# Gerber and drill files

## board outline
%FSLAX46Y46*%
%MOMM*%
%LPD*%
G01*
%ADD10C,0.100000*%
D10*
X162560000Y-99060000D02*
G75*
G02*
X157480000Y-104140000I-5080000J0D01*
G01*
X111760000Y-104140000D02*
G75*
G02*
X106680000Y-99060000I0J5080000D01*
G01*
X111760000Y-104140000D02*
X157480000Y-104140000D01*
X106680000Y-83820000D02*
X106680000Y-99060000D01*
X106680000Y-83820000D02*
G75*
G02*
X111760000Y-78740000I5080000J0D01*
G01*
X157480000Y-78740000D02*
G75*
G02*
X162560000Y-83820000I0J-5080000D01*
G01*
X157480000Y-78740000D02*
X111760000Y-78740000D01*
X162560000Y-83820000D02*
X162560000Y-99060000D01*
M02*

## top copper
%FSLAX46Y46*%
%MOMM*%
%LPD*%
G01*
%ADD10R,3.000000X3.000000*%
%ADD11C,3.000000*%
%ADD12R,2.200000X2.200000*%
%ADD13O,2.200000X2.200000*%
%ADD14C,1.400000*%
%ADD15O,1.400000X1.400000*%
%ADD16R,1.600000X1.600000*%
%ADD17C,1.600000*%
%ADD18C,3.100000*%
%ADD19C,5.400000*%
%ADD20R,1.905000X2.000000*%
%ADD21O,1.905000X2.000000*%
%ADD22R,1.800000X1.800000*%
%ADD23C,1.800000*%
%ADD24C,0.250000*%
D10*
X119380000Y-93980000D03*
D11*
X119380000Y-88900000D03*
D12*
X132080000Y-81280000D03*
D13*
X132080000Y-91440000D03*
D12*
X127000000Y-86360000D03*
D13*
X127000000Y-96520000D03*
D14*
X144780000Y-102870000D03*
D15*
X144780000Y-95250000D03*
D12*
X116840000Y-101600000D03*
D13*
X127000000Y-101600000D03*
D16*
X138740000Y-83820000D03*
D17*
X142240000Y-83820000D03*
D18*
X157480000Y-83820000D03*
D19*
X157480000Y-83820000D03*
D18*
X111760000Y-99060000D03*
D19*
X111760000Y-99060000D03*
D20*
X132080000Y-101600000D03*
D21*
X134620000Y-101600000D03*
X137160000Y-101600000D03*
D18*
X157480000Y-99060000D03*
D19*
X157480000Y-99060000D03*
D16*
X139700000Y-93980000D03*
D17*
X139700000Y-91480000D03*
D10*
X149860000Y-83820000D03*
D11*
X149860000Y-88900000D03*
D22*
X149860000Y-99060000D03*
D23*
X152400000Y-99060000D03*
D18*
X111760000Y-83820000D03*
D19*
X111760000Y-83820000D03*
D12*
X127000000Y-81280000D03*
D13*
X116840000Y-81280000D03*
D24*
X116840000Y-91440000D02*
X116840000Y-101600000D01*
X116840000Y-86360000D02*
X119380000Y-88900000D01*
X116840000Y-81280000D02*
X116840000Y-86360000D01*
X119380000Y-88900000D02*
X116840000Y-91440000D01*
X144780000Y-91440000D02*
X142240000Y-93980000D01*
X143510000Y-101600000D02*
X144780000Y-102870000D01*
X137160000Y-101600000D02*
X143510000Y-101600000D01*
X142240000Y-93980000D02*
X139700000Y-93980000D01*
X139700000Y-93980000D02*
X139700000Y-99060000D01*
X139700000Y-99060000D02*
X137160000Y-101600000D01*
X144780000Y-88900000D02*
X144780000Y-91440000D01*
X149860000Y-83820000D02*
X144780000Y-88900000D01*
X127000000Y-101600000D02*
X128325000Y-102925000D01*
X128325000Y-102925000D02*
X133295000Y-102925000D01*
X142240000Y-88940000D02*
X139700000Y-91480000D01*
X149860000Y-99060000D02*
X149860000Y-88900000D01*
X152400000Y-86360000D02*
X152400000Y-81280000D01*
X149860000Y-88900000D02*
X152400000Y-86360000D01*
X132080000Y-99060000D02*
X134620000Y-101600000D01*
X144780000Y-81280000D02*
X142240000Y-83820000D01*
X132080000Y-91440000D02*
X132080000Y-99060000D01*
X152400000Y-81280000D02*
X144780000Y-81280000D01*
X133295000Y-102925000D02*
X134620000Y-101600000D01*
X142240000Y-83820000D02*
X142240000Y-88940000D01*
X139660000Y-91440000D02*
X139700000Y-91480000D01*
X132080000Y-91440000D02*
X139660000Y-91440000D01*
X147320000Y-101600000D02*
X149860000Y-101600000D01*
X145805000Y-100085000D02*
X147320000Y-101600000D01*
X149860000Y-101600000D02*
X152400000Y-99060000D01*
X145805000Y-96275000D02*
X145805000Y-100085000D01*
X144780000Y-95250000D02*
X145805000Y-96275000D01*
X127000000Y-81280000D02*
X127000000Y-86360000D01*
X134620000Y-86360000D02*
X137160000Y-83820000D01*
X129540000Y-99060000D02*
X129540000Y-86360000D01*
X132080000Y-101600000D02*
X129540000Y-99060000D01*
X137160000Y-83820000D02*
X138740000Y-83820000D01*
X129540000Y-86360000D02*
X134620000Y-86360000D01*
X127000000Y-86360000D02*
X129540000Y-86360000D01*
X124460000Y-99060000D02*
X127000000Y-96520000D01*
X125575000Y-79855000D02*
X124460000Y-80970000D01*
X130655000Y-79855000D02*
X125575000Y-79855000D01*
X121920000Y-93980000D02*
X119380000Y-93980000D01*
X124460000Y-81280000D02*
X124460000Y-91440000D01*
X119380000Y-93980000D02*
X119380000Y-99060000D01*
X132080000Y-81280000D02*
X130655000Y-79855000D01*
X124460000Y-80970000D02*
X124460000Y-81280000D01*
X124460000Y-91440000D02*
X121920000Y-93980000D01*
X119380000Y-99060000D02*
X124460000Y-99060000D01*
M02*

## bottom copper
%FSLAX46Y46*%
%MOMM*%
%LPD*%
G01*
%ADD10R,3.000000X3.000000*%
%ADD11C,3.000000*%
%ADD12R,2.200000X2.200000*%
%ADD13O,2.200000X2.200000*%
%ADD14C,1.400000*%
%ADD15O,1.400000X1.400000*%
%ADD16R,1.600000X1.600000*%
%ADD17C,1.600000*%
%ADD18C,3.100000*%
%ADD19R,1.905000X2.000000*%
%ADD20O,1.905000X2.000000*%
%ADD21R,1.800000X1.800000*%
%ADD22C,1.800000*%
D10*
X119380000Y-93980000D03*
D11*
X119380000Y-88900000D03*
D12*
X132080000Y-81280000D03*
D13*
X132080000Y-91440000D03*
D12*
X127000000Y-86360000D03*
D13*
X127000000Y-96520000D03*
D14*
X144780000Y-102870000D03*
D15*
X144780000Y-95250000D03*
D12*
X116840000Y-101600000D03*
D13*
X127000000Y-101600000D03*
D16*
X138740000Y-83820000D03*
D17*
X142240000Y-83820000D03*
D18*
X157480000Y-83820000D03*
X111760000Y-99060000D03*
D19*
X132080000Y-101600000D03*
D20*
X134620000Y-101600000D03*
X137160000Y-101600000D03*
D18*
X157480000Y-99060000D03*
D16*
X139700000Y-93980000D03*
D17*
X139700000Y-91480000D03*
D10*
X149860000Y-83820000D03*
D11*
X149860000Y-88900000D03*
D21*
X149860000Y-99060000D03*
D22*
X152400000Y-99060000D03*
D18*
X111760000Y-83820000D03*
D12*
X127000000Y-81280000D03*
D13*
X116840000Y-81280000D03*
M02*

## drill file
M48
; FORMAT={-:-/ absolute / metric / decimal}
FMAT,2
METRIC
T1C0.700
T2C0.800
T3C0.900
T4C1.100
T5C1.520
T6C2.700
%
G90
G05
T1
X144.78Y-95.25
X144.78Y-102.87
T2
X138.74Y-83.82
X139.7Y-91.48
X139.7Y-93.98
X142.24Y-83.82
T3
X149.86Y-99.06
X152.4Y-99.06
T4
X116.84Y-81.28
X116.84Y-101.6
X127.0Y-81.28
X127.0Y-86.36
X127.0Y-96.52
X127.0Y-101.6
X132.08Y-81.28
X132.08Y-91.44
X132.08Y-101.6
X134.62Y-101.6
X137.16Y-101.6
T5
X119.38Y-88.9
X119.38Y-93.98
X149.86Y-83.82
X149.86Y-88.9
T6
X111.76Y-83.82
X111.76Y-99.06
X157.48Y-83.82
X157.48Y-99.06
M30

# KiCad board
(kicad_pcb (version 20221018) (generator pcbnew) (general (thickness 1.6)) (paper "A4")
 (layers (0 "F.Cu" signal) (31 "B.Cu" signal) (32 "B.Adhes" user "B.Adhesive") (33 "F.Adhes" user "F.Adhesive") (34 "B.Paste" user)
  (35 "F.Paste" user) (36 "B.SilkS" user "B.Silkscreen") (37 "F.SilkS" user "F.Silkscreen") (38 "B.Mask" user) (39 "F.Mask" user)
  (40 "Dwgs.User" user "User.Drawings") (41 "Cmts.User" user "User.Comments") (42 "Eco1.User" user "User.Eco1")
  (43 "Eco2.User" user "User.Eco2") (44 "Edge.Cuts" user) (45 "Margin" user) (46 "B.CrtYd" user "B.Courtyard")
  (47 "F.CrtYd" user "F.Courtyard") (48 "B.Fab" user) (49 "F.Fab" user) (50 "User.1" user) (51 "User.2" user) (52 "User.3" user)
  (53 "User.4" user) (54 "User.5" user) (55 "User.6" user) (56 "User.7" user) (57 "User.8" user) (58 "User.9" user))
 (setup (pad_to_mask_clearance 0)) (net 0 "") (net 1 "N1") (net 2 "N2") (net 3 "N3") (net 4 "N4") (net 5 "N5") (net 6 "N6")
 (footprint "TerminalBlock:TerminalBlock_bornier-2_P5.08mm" (layer "F.Cu") (at 119.38 93.98 90)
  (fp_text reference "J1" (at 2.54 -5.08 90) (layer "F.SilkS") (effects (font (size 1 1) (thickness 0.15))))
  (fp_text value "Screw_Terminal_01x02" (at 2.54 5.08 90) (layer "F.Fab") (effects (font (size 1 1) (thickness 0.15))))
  (pad "1" thru_hole rect (at 0 0 90) (size 3 3) (drill 1.52) (layers "*.Cu" "*.Mask") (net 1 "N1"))
  (pad "2" thru_hole circle (at 5.08 0 90) (size 3 3) (drill 1.52) (layers "*.Cu" "*.Mask") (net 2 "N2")))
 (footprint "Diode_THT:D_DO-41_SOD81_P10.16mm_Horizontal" (layer "F.Cu") (at 132.08 81.28 -90)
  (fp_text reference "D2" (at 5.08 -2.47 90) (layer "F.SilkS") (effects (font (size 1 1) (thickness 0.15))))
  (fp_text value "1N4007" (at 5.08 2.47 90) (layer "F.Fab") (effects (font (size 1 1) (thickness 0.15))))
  (pad "1" thru_hole rect (at 0 0 270) (size 2.2 2.2) (drill 1.1) (layers "*.Cu" "*.Mask") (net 1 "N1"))
  (pad "2" thru_hole oval (at 10.16 0 270) (size 2.2 2.2) (drill 1.1) (layers "*.Cu" "*.Mask") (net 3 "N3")))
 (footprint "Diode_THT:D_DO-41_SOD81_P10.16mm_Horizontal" (layer "F.Cu") (at 127 86.36 -90)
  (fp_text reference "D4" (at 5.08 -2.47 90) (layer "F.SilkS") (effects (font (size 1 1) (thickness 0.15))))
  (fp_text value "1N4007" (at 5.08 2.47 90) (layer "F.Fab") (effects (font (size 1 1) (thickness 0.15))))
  (pad "1" thru_hole rect (at 0 0 270) (size 2.2 2.2) (drill 1.1) (layers "*.Cu" "*.Mask") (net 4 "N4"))
  (pad "2" thru_hole oval (at 10.16 0 270) (size 2.2 2.2) (drill 1.1) (layers "*.Cu" "*.Mask") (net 1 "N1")))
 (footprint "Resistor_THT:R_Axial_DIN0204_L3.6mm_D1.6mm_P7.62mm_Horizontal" (layer "F.Cu") (at 144.78 102.87 90)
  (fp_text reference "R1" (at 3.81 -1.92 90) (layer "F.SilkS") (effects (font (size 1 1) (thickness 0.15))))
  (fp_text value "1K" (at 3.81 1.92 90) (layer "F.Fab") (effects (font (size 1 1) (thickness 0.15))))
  (pad "1" thru_hole circle (at 0 0 90) (size 1.4 1.4) (drill 0.7) (layers "*.Cu" "*.Mask") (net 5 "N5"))
  (pad "2" thru_hole oval (at 7.62 0 90) (size 1.4 1.4) (drill 0.7) (layers "*.Cu" "*.Mask") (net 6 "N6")))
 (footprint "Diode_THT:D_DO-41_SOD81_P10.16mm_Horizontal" (layer "F.Cu") (at 116.84 101.6)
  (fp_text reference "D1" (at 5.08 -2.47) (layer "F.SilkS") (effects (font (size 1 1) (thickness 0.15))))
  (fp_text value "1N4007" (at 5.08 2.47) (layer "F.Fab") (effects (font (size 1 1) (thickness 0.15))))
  (pad "1" thru_hole rect (at 0 0) (size 2.2 2.2) (drill 1.1) (layers "*.Cu" "*.Mask") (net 2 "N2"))
  (pad "2" thru_hole oval (at 10.16 0) (size 2.2 2.2) (drill 1.1) (layers "*.Cu" "*.Mask") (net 3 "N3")))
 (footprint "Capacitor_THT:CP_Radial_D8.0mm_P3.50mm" (layer "F.Cu") (at 138.74 83.82)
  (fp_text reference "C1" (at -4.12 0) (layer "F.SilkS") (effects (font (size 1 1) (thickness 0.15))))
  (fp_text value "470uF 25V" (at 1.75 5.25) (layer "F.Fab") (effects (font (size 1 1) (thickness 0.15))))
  (pad "1" thru_hole rect (at 0 0) (size 1.6 1.6) (drill 0.8) (layers "*.Cu" "*.Mask") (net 4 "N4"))
  (pad "2" thru_hole circle (at 3.5 0) (size 1.6 1.6) (drill 0.8) (layers "*.Cu" "*.Mask") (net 3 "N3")))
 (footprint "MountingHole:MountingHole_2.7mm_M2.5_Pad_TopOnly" (layer "F.Cu") (at 157.48 83.82)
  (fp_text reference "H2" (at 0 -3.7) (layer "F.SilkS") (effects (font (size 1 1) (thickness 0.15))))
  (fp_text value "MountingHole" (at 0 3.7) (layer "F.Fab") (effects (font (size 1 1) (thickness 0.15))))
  (pad "1" thru_hole circle (at 0 0) (size 3.1 3.1) (drill 2.7) (layers "*.Cu" "*.Mask"))
  (pad "1" connect circle (at 0 0) (size 5.4 5.4) (layers "F.Cu" "F.Mask")))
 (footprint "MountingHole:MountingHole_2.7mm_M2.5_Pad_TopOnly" (layer "F.Cu") (at 111.76 99.06)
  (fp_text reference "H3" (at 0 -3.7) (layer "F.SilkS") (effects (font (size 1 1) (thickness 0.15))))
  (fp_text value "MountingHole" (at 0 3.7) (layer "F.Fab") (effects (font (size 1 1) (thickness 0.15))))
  (pad "1" thru_hole circle (at 0 0) (size 3.1 3.1) (drill 2.7) (layers "*.Cu" "*.Mask"))
  (pad "1" connect circle (at 0 0) (size 5.4 5.4) (layers "F.Cu" "F.Mask")))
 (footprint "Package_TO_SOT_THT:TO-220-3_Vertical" (layer "F.Cu") (at 132.08 101.6)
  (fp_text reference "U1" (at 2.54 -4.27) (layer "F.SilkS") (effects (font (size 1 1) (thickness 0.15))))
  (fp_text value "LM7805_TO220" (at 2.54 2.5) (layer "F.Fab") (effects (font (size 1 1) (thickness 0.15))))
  (pad "1" thru_hole rect (at 0 0) (size 1.905 2) (drill 1.1) (layers "*.Cu" "*.Mask") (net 4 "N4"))
  (pad "2" thru_hole oval (at 2.54 0) (size 1.905 2) (drill 1.1) (layers "*.Cu" "*.Mask") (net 3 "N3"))
  (pad "3" thru_hole oval (at 5.08 0) (size 1.905 2) (drill 1.1) (layers "*.Cu" "*.Mask") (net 5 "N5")))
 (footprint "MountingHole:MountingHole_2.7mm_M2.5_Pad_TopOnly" (layer "F.Cu") (at 157.48 99.06)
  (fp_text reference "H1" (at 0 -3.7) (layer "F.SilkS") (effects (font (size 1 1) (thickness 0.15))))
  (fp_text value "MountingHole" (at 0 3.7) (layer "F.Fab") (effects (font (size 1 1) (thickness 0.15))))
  (pad "1" thru_hole circle (at 0 0) (size 3.1 3.1) (drill 2.7) (layers "*.Cu" "*.Mask"))
  (pad "1" connect circle (at 0 0) (size 5.4 5.4) (layers "F.Cu" "F.Mask")))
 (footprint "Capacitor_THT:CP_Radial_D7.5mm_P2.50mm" (layer "F.Cu") (at 139.7 93.98 90)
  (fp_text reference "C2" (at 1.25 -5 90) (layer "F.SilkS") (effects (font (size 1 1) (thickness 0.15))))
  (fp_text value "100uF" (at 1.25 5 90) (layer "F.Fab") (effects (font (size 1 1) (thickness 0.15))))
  (pad "1" thru_hole rect (at 0 0 90) (size 1.6 1.6) (drill 0.8) (layers "*.Cu" "*.Mask") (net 5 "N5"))
  (pad "2" thru_hole circle (at 2.5 0 90) (size 1.6 1.6) (drill 0.8) (layers "*.Cu" "*.Mask") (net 3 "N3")))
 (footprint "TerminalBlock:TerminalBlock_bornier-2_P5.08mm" (layer "F.Cu") (at 149.86 83.82 -90)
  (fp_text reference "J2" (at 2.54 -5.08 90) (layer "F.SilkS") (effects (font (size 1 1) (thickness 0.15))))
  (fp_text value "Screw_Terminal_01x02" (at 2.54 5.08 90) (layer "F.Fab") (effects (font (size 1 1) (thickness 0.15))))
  (pad "1" thru_hole rect (at 0 0 270) (size 3 3) (drill 1.52) (layers "*.Cu" "*.Mask") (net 5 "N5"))
  (pad "2" thru_hole circle (at 5.08 0 270) (size 3 3) (drill 1.52) (layers "*.Cu" "*.Mask") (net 3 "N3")))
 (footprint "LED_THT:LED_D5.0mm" (layer "F.Cu") (at 149.86 99.06)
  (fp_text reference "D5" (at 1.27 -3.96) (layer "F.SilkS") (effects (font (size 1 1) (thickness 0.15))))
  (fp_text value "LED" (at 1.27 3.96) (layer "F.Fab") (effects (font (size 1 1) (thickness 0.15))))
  (pad "1" thru_hole rect (at 0 0) (size 1.8 1.8) (drill 0.9) (layers "*.Cu" "*.Mask") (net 3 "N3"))
  (pad "2" thru_hole circle (at 2.54 0) (size 1.8 1.8) (drill 0.9) (layers "*.Cu" "*.Mask") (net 6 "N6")))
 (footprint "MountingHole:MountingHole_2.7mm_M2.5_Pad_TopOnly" (layer "F.Cu") (at 111.76 83.82)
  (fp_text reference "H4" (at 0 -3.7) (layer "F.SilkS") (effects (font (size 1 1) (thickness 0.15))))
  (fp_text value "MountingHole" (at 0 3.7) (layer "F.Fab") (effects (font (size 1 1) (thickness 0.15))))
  (pad "1" thru_hole circle (at 0 0) (size 3.1 3.1) (drill 2.7) (layers "*.Cu" "*.Mask"))
  (pad "1" connect circle (at 0 0) (size 5.4 5.4) (layers "F.Cu" "F.Mask")))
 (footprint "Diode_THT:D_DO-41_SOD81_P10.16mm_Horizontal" (layer "F.Cu") (at 127 81.28 180)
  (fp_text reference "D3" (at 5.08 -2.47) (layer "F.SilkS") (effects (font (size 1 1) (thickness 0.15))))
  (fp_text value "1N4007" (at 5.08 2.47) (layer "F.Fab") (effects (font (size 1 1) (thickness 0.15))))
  (pad "1" thru_hole rect (at 0 0 180) (size 2.2 2.2) (drill 1.1) (layers "*.Cu" "*.Mask") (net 4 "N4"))
  (pad "2" thru_hole oval (at 10.16 0 180) (size 2.2 2.2) (drill 1.1) (layers "*.Cu" "*.Mask") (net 2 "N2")))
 (gr_arc (start 162.56 99.06) (mid 161.072102 102.652102) (end 157.48 104.14) (stroke (width 0.1) (type default)) (layer "Edge.Cuts"))
 (gr_arc (start 111.76 104.14) (mid 108.167898 102.652102) (end 106.68 99.06) (stroke (width 0.1) (type default)) (layer "Edge.Cuts"))
 (gr_line (start 111.76 104.14) (end 157.48 104.14) (stroke (width 0.1) (type default)) (layer "Edge.Cuts"))
 (gr_line (start 106.68 83.82) (end 106.68 99.06) (stroke (width 0.1) (type default)) (layer "Edge.Cuts"))
 (gr_arc (start 106.68 83.82) (mid 108.167898 80.227898) (end 111.76 78.74) (stroke (width 0.1) (type default)) (layer "Edge.Cuts"))
 (gr_arc (start 157.48 78.74) (mid 161.072102 80.227898) (end 162.56 83.82) (stroke (width 0.1) (type default)) (layer "Edge.Cuts"))
 (gr_line (start 157.48 78.74) (end 111.76 78.74) (stroke (width 0.1) (type default)) (layer "Edge.Cuts"))
 (gr_line (start 162.56 83.82) (end 162.56 99.06) (stroke (width 0.1) (type default)) (layer "Edge.Cuts"))
 (segment (start 116.84 91.44) (end 116.84 101.6) (width 0.25) (layer "F.Cu") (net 2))
 (segment (start 116.84 86.36) (end 119.38 88.9) (width 0.25) (layer "F.Cu") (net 2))
 (segment (start 116.84 81.28) (end 116.84 86.36) (width 0.25) (layer "F.Cu") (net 2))
 (segment (start 119.38 88.9) (end 116.84 91.44) (width 0.25) (layer "F.Cu") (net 2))
 (segment (start 144.78 91.44) (end 142.24 93.98) (width 0.25) (layer "F.Cu") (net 5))
 (segment (start 143.51 101.6) (end 144.78 102.87) (width 0.25) (layer "F.Cu") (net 5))
 (segment (start 137.16 101.6) (end 143.51 101.6) (width 0.25) (layer "F.Cu") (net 5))
 (segment (start 142.24 93.98) (end 139.7 93.98) (width 0.25) (layer "F.Cu") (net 5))
 (segment (start 139.7 93.98) (end 139.7 99.06) (width 0.25) (layer "F.Cu") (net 5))
 (segment (start 139.7 99.06) (end 137.16 101.6) (width 0.25) (layer "F.Cu") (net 5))
 (segment (start 144.78 88.9) (end 144.78 91.44) (width 0.25) (layer "F.Cu") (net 5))
 (segment (start 149.86 83.82) (end 144.78 88.9) (width 0.25) (layer "F.Cu") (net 5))
 (segment (start 127 101.6) (end 128.325 102.925) (width 0.25) (layer "F.Cu") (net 3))
 (segment (start 128.325 102.925) (end 133.295 102.925) (width 0.25) (layer "F.Cu") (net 3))
 (segment (start 142.24 88.94) (end 139.7 91.48) (width 0.25) (layer "F.Cu") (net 3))
 (segment (start 149.86 99.06) (end 149.86 88.9) (width 0.25) (layer "F.Cu") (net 3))
 (segment (start 152.4 86.36) (end 152.4 81.28) (width 0.25) (layer "F.Cu") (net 3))
 (segment (start 149.86 88.9) (end 152.4 86.36) (width 0.25) (layer "F.Cu") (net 3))
 (segment (start 132.08 99.06) (end 134.62 101.6) (width 0.25) (layer "F.Cu") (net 3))
 (segment (start 144.78 81.28) (end 142.24 83.82) (width 0.25) (layer "F.Cu") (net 3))
 (segment (start 132.08 91.44) (end 132.08 99.06) (width 0.25) (layer "F.Cu") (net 3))
 (segment (start 152.4 81.28) (end 144.78 81.28) (width 0.25) (layer "F.Cu") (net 3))
 (segment (start 133.295 102.925) (end 134.62 101.6) (width 0.25) (layer "F.Cu") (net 3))
 (segment (start 142.24 83.82) (end 142.24 88.94) (width 0.25) (layer "F.Cu") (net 3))
 (segment (start 139.66 91.44) (end 139.7 91.48) (width 0.25) (layer "F.Cu") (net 3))
 (segment (start 132.08 91.44) (end 139.66 91.44) (width 0.25) (layer "F.Cu") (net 3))
 (segment (start 147.32 101.6) (end 149.86 101.6) (width 0.25) (layer "F.Cu") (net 6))
 (segment (start 145.805 100.085) (end 147.32 101.6) (width 0.25) (layer "F.Cu") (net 6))
 (segment (start 149.86 101.6) (end 152.4 99.06) (width 0.25) (layer "F.Cu") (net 6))
 (segment (start 145.805 96.275) (end 145.805 100.085) (width 0.25) (layer "F.Cu") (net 6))
 (segment (start 144.78 95.25) (end 145.805 96.275) (width 0.25) (layer "F.Cu") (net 6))
 (segment (start 127 81.28) (end 127 86.36) (width 0.25) (layer "F.Cu") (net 4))
 (segment (start 134.62 86.36) (end 137.16 83.82) (width 0.25) (layer "F.Cu") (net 4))
 (segment (start 129.54 99.06) (end 129.54 86.36) (width 0.25) (layer "F.Cu") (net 4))
 (segment (start 132.08 101.6) (end 129.54 99.06) (width 0.25) (layer "F.Cu") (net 4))
 (segment (start 137.16 83.82) (end 138.74 83.82) (width 0.25) (layer "F.Cu") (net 4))
 (segment (start 129.54 86.36) (end 134.62 86.36) (width 0.25) (layer "F.Cu") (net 4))
 (segment (start 127 86.36) (end 129.54 86.36) (width 0.25) (layer "F.Cu") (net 4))
 (segment (start 124.46 99.06) (end 127 96.52) (width 0.25) (layer "F.Cu") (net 1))
 (segment (start 125.575 79.855) (end 124.46 80.97) (width 0.25) (layer "F.Cu") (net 1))
 (segment (start 130.655 79.855) (end 125.575 79.855) (width 0.25) (layer "F.Cu") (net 1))
 (segment (start 121.92 93.98) (end 119.38 93.98) (width 0.25) (layer "F.Cu") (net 1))
 (segment (start 124.46 81.28) (end 124.46 91.44) (width 0.25) (layer "F.Cu") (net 1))
 (segment (start 119.38 93.98) (end 119.38 99.06) (width 0.25) (layer "F.Cu") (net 1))
 (segment (start 132.08 81.28) (end 130.655 79.855) (width 0.25) (layer "F.Cu") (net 1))
 (segment (start 124.46 80.97) (end 124.46 81.28) (width 0.25) (layer "F.Cu") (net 1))
 (segment (start 124.46 91.44) (end 121.92 93.98) (width 0.25) (layer "F.Cu") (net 1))
 (segment (start 119.38 99.06) (end 124.46 99.06) (width 0.25) (layer "F.Cu") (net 1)))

